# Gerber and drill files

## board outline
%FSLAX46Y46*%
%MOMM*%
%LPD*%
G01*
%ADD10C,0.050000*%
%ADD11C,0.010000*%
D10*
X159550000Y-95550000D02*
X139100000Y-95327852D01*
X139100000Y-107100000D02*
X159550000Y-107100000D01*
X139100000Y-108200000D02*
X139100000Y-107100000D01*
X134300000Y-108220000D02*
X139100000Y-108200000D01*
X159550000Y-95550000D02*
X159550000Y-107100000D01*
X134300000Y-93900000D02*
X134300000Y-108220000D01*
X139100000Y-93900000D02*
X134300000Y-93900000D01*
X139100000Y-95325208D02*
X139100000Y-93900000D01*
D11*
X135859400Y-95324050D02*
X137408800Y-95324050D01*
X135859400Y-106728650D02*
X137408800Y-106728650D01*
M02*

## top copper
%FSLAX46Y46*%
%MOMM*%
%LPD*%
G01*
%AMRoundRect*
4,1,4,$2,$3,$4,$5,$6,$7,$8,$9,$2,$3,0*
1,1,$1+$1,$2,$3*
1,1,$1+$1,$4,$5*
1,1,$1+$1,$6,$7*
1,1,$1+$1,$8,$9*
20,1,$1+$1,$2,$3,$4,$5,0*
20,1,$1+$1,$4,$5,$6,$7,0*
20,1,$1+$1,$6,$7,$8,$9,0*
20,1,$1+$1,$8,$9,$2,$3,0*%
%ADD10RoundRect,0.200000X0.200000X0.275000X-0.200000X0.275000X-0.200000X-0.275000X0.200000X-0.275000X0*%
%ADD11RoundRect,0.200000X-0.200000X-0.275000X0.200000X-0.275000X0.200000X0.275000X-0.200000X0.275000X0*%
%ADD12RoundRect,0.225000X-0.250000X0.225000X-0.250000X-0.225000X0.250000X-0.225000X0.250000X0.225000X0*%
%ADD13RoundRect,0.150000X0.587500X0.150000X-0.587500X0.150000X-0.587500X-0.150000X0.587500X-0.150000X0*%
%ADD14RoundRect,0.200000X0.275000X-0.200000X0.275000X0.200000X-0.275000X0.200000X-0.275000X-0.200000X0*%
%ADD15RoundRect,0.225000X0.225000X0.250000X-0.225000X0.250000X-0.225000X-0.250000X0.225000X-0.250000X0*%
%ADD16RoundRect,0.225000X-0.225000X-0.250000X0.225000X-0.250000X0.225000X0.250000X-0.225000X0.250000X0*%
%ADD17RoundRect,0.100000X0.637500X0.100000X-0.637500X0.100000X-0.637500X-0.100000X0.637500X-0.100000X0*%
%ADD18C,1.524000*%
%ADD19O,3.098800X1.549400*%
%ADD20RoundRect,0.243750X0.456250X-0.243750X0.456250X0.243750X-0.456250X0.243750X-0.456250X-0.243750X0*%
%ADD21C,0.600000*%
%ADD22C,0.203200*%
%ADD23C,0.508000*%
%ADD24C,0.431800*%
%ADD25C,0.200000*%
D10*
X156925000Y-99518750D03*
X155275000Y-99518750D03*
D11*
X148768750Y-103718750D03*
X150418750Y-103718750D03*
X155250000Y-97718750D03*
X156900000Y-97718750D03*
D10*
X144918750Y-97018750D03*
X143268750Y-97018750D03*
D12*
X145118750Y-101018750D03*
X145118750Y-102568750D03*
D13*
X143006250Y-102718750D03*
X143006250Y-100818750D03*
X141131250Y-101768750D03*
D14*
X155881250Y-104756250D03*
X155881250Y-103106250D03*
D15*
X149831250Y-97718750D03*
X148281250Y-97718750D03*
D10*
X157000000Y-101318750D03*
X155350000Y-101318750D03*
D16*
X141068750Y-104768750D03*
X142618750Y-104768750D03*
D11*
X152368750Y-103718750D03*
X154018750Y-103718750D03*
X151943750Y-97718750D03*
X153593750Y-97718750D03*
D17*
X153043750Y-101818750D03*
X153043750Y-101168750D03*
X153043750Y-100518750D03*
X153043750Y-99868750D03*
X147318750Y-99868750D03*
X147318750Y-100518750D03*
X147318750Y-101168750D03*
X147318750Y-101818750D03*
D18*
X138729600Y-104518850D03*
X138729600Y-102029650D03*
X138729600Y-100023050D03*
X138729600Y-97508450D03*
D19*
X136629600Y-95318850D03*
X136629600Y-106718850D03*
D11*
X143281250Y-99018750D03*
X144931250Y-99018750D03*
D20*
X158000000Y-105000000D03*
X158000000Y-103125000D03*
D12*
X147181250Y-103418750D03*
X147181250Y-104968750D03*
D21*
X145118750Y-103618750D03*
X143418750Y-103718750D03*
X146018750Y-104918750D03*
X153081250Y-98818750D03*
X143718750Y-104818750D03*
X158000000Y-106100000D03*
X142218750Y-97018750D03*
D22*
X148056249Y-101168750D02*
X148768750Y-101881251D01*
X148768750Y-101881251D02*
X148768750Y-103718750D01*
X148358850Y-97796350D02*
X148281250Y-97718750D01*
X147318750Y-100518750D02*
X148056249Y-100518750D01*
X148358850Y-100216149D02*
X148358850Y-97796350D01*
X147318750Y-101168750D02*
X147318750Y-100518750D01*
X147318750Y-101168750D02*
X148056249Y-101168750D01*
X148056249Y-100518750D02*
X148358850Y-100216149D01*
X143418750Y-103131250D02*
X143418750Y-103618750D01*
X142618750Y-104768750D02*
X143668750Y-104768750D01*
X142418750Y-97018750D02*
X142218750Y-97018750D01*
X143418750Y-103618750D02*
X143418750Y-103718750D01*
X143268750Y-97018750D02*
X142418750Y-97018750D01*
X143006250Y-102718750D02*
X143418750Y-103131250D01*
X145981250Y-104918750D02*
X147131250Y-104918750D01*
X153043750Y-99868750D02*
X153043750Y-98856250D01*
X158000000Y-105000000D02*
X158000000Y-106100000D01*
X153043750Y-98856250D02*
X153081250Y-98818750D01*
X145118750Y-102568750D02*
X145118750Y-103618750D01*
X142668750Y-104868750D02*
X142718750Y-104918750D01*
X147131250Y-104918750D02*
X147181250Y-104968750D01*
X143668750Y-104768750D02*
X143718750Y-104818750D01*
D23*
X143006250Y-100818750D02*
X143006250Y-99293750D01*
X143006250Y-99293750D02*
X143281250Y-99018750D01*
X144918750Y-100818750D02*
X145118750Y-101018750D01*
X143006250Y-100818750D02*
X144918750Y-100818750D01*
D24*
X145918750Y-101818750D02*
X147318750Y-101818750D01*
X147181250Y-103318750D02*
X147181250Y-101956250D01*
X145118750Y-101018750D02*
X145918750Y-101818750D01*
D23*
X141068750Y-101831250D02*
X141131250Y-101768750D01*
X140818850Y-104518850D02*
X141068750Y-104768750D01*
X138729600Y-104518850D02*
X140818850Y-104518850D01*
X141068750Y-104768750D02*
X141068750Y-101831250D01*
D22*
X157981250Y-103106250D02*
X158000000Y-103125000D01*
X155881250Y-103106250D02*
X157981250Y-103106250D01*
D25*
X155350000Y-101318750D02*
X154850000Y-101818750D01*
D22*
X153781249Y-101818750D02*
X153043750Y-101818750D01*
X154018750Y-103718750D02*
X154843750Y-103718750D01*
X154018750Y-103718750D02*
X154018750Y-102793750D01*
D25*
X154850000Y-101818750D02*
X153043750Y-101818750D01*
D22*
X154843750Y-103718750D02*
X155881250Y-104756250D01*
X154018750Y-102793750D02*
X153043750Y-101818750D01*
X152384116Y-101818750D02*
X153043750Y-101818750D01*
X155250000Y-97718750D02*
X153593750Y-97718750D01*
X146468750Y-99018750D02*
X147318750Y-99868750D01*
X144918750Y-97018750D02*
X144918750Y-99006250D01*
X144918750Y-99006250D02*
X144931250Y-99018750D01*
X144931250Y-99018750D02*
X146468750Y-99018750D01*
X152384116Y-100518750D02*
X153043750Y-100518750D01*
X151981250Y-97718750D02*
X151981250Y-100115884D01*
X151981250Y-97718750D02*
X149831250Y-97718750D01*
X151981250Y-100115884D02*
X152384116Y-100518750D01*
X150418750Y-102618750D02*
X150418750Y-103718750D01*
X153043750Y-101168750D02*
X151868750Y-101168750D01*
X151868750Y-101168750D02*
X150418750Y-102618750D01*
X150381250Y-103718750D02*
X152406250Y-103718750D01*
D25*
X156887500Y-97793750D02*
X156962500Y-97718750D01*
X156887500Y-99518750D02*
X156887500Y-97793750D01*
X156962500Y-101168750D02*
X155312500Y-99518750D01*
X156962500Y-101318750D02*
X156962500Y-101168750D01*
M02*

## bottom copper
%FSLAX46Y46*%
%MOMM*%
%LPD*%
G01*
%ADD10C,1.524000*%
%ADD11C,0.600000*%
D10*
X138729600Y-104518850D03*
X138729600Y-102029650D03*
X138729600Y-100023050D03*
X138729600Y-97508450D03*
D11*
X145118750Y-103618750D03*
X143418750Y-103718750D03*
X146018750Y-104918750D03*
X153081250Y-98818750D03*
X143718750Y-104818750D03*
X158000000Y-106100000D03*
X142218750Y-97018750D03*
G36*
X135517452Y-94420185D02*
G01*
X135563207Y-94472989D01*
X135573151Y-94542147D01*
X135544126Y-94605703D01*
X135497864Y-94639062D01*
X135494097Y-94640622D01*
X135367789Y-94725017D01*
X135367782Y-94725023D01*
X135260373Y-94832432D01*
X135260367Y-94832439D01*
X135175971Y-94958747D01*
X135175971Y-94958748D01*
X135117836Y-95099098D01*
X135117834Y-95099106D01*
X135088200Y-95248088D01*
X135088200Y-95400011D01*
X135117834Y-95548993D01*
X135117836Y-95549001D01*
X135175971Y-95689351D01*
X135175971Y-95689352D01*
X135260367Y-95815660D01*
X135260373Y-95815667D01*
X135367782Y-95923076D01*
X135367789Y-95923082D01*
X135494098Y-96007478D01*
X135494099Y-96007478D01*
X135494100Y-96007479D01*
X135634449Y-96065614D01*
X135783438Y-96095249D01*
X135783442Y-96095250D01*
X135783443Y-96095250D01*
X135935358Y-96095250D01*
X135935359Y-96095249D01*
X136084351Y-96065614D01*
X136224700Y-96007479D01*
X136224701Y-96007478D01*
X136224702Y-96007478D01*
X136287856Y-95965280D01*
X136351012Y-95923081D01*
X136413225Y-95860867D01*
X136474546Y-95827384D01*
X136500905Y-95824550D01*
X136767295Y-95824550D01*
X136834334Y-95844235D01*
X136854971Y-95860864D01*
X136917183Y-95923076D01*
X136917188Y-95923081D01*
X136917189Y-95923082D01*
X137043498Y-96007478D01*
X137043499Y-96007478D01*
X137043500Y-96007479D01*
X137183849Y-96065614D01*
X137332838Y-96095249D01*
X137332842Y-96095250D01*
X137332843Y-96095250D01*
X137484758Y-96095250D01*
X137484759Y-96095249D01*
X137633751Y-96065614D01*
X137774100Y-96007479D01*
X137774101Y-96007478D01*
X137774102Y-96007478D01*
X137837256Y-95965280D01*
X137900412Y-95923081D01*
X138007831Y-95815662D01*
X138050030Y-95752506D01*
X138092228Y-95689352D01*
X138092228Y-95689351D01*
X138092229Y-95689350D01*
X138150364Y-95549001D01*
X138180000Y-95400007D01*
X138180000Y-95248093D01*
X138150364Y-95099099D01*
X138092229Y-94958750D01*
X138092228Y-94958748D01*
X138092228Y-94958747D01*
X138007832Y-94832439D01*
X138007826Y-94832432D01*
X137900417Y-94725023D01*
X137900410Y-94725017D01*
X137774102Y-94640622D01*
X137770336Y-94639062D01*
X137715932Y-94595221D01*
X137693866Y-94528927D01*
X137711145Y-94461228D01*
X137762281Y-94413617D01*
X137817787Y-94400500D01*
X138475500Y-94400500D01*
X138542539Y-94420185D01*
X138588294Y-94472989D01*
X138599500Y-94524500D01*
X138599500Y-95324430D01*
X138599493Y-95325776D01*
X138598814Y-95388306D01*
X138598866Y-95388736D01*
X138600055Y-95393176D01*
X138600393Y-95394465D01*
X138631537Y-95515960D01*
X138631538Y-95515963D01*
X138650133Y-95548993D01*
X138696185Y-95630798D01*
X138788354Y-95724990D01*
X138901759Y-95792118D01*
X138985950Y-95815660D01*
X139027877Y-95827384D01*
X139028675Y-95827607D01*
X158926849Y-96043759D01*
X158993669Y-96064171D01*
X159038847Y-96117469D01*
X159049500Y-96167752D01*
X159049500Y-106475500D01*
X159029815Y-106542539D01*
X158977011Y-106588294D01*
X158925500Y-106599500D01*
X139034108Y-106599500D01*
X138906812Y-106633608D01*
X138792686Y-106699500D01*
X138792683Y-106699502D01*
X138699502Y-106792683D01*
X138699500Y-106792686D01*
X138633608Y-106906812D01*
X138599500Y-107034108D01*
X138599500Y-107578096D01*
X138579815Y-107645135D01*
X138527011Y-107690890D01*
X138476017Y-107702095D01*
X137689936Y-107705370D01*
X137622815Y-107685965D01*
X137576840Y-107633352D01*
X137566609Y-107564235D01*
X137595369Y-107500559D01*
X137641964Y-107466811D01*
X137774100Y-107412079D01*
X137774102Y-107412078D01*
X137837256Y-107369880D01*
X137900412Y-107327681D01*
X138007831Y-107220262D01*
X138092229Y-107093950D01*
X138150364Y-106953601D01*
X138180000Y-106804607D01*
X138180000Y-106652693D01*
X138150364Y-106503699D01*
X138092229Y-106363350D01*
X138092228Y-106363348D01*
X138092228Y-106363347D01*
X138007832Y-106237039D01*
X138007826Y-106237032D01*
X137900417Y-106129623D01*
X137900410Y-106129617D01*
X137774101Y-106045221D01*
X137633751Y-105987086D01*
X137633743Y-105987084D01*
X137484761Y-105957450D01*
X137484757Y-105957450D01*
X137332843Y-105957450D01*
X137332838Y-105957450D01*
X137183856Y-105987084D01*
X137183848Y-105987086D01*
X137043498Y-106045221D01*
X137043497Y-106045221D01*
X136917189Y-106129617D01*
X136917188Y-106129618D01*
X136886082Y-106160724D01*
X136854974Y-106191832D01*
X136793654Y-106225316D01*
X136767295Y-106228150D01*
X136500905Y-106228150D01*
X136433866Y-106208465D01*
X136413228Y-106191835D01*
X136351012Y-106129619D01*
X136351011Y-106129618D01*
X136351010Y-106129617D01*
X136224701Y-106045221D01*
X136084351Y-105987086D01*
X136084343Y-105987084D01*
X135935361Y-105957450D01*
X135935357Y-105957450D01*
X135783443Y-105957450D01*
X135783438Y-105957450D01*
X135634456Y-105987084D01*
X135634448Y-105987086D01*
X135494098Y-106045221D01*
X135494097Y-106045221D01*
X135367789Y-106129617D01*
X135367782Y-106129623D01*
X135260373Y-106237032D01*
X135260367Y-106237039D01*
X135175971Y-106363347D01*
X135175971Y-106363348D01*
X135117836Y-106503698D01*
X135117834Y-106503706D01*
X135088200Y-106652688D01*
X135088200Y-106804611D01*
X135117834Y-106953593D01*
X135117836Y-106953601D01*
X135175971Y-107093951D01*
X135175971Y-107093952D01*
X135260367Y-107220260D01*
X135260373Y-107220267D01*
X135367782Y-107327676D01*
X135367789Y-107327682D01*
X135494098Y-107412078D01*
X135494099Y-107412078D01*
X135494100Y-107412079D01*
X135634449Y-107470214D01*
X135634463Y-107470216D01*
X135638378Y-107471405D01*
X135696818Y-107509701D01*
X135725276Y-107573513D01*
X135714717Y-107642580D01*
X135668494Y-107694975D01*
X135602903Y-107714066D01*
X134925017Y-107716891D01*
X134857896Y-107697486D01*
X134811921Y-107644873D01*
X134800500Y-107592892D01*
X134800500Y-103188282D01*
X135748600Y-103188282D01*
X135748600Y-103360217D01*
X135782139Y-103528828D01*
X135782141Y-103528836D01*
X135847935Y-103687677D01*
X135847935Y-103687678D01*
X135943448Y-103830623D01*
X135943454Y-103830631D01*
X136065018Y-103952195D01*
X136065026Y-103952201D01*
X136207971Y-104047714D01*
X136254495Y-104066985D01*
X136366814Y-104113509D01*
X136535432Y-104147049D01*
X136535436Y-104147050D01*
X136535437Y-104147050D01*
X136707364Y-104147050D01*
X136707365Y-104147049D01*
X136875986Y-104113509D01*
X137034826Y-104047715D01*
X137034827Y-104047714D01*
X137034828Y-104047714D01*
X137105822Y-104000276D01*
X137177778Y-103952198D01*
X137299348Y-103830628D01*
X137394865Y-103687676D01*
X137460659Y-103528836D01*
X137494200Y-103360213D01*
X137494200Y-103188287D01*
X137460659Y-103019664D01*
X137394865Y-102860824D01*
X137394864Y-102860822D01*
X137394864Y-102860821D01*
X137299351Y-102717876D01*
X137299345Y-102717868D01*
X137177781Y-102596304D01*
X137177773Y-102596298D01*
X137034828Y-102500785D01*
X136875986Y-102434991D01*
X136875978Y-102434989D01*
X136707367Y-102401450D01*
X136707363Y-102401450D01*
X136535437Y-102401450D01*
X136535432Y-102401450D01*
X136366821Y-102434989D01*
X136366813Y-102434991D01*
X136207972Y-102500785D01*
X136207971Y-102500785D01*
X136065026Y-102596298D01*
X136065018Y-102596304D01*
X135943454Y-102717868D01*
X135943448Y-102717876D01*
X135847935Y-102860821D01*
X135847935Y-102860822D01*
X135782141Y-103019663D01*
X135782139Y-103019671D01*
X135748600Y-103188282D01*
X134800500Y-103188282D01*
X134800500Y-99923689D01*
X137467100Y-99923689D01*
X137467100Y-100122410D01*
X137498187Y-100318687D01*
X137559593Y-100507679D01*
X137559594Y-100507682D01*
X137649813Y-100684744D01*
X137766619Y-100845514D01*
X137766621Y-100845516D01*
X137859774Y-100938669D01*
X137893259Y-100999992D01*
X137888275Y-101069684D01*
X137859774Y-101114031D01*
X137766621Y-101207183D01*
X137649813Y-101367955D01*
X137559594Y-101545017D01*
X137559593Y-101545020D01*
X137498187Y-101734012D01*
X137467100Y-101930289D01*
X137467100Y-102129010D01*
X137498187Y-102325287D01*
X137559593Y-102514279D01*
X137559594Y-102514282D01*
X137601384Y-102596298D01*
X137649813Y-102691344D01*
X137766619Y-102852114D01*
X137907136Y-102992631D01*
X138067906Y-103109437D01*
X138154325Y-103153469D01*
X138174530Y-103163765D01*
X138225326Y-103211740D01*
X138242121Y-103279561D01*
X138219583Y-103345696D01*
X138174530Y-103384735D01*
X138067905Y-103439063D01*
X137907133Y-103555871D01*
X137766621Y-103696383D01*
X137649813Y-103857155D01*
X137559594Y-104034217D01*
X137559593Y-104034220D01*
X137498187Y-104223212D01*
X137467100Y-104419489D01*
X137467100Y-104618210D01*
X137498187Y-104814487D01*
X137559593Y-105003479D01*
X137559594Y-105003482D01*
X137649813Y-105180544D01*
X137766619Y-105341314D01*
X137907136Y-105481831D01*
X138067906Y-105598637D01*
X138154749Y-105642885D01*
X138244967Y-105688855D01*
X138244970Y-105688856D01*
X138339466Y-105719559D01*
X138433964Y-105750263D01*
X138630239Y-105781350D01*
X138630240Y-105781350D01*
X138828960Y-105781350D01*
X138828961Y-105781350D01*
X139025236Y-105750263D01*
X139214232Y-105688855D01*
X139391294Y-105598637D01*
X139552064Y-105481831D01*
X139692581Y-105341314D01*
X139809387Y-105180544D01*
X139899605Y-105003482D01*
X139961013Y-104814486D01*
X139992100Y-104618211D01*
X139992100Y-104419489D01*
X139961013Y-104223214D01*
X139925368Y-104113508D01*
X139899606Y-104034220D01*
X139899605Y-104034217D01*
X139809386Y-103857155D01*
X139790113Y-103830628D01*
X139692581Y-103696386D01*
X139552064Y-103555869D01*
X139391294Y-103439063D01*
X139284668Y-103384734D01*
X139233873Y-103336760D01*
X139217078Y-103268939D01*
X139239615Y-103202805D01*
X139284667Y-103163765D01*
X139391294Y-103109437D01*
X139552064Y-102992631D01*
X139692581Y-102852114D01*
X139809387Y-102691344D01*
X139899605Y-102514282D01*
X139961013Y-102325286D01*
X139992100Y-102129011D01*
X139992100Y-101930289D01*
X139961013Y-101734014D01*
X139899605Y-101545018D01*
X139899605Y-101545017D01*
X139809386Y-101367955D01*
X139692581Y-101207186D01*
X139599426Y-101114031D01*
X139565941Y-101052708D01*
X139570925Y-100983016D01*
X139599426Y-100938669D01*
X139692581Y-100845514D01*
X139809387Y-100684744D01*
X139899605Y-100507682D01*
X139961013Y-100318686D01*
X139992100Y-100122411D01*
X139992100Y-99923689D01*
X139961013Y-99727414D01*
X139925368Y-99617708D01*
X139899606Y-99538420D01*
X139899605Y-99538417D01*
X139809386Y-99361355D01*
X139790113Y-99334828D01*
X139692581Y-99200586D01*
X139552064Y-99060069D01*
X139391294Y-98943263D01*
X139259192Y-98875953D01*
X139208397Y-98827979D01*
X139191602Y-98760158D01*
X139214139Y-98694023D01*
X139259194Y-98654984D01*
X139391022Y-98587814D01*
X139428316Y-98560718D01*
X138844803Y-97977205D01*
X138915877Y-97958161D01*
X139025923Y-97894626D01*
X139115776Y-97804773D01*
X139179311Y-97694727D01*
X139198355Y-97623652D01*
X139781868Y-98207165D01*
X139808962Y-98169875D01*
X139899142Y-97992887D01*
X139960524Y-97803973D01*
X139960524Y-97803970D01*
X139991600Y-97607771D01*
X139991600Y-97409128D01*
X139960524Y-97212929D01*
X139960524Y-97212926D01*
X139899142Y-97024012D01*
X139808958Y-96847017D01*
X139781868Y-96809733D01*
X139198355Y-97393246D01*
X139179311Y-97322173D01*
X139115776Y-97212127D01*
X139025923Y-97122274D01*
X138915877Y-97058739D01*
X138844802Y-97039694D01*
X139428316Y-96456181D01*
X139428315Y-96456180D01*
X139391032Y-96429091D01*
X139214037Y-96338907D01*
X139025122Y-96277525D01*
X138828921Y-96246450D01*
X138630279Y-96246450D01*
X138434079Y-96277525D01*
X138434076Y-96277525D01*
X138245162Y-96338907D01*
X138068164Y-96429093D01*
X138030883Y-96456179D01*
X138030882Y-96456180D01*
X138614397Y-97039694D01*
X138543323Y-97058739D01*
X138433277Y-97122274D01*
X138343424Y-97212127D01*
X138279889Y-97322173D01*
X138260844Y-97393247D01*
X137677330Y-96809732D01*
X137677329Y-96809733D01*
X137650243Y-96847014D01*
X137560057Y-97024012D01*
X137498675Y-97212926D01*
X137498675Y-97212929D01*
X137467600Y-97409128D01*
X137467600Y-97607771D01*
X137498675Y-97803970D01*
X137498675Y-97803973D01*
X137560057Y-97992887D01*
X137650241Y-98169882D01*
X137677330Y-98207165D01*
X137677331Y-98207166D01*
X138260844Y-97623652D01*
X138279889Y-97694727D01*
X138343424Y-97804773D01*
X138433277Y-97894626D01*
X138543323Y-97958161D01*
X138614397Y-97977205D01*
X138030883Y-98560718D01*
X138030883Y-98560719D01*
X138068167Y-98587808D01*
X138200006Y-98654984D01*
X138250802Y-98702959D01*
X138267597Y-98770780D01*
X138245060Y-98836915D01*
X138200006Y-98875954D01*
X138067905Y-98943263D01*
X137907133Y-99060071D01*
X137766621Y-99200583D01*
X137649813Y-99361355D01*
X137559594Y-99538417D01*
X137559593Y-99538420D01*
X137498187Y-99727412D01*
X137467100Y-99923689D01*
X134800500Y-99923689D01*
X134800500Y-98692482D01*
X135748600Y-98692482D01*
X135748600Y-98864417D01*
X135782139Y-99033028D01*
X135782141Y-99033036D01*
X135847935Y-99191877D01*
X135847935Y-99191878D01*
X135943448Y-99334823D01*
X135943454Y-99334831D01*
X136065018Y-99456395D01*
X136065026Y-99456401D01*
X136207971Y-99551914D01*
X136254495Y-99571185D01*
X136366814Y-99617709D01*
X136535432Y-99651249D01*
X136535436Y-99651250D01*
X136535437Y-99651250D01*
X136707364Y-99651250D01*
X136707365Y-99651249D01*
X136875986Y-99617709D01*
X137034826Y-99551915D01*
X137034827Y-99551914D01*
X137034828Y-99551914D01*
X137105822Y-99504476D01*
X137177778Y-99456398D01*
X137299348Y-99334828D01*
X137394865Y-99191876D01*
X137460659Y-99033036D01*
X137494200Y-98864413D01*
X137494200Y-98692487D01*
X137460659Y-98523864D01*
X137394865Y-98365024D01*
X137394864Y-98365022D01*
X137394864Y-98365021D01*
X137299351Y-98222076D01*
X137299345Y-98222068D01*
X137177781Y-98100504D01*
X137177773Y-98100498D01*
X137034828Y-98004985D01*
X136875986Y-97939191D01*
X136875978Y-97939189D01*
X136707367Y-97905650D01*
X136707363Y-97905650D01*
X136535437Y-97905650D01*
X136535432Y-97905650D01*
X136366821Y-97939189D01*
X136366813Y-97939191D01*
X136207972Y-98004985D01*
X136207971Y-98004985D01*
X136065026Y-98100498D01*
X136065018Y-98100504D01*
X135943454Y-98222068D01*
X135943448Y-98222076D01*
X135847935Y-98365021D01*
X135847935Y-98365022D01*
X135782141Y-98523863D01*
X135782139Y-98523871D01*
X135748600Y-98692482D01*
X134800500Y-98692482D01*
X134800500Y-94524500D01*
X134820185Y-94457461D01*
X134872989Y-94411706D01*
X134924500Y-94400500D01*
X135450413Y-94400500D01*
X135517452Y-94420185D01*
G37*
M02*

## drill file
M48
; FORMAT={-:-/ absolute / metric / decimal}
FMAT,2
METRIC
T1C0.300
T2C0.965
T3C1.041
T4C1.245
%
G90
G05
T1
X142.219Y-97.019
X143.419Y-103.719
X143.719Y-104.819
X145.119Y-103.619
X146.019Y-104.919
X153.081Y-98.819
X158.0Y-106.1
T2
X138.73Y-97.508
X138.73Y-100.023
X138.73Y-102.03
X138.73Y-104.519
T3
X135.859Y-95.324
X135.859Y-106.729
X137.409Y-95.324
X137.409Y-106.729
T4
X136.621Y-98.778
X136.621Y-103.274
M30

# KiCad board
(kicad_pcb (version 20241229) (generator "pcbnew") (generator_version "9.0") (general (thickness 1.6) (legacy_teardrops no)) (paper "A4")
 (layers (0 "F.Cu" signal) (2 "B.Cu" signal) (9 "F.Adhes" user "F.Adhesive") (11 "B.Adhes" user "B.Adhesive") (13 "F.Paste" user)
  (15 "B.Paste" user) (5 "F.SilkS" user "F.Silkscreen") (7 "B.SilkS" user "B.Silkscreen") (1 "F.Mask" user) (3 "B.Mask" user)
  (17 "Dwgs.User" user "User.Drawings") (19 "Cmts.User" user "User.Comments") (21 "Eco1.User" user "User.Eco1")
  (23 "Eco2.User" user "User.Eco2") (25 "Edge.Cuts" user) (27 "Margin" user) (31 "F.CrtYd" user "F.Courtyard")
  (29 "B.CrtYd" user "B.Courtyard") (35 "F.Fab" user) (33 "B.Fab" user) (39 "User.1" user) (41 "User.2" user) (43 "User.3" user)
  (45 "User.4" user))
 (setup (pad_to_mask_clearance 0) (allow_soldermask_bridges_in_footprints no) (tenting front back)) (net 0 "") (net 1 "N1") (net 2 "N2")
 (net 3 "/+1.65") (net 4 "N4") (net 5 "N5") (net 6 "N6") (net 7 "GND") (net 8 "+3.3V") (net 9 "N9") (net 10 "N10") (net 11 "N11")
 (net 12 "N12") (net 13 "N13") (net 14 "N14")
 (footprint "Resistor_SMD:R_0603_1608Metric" (layer "F.Cu") (at 156.1 99.51875 180)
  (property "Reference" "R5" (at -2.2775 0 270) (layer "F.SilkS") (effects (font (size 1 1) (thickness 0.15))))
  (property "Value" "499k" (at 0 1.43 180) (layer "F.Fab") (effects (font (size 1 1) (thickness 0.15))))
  (pad "1" smd roundrect (at -0.825 0 180) (size 0.8 0.95) (layers "F.Cu" "F.Mask" "F.Paste") (roundrect_rratio 0.25) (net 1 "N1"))
  (pad "2" smd roundrect (at 0.825 0 180) (size 0.8 0.95) (layers "F.Cu" "F.Mask" "F.Paste") (roundrect_rratio 0.25) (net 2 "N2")))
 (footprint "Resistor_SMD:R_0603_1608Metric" (layer "F.Cu") (at 149.59375 103.71875)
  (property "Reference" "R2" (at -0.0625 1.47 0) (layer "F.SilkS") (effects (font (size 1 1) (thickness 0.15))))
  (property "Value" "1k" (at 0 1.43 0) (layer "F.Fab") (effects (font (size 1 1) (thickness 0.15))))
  (pad "1" smd roundrect (at -0.825 0) (size 0.8 0.95) (layers "F.Cu" "F.Mask" "F.Paste") (roundrect_rratio 0.25) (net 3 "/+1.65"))
  (pad "2" smd roundrect (at 0.825 0) (size 0.8 0.95) (layers "F.Cu" "F.Mask" "F.Paste") (roundrect_rratio 0.25) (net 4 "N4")))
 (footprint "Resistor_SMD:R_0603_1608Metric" (layer "F.Cu") (at 156.075 97.71875)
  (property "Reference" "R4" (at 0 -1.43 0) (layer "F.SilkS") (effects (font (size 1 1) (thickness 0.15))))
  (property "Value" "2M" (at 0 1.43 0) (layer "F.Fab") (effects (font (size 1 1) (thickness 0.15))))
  (pad "1" smd roundrect (at -0.825 0) (size 0.8 0.95) (layers "F.Cu" "F.Mask" "F.Paste") (roundrect_rratio 0.25) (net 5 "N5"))
  (pad "2" smd roundrect (at 0.825 0) (size 0.8 0.95) (layers "F.Cu" "F.Mask" "F.Paste") (roundrect_rratio 0.25) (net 1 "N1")))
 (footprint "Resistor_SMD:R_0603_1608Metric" (layer "F.Cu") (at 144.09375 97.01875 180)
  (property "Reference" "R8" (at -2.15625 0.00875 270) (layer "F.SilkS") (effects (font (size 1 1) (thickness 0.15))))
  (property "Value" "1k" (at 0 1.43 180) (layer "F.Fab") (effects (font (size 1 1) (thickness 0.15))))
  (pad "1" smd roundrect (at -0.825 0 180) (size 0.8 0.95) (layers "F.Cu" "F.Mask" "F.Paste") (roundrect_rratio 0.25) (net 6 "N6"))
  (pad "2" smd roundrect (at 0.825 0 180) (size 0.8 0.95) (layers "F.Cu" "F.Mask" "F.Paste") (roundrect_rratio 0.25) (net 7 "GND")))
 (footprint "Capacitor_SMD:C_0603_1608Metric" (layer "F.Cu") (at 145.11875 101.79375 -90)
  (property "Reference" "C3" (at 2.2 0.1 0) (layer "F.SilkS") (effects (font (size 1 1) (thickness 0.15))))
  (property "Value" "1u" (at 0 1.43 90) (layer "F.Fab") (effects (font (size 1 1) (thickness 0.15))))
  (pad "1" smd roundrect (at -0.775 0 270) (size 0.9 0.95) (layers "F.Cu" "F.Mask" "F.Paste") (roundrect_rratio 0.25) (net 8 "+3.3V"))
  (pad "2" smd roundrect (at 0.775 0 270) (size 0.9 0.95) (layers "F.Cu" "F.Mask" "F.Paste") (roundrect_rratio 0.25) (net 7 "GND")))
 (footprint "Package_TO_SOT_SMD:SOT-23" (layer "F.Cu") (at 142.06875 101.76875 180)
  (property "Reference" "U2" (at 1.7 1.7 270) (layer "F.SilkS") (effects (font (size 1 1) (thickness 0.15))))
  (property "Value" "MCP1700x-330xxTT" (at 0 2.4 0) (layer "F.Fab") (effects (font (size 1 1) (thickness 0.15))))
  (pad "1" smd roundrect (at -0.9375 -0.95 180) (size 1.475 0.6) (layers "F.Cu" "F.Mask" "F.Paste") (roundrect_rratio 0.25) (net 7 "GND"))
  (pad "2" smd roundrect (at -0.9375 0.95 180) (size 1.475 0.6) (layers "F.Cu" "F.Mask" "F.Paste") (roundrect_rratio 0.25) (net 8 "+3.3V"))
  (pad "3" smd roundrect (at 0.9375 0 180) (size 1.475 0.6) (layers "F.Cu" "F.Mask" "F.Paste") (roundrect_rratio 0.25) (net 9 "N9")))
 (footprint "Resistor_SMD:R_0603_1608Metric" (layer "F.Cu") (at 155.88125 103.93125 90)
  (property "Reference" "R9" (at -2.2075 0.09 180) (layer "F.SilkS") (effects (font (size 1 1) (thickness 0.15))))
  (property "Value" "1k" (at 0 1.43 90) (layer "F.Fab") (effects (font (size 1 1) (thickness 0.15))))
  (pad "1" smd roundrect (at -0.825 0 90) (size 0.8 0.95) (layers "F.Cu" "F.Mask" "F.Paste") (roundrect_rratio 0.25) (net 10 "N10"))
  (pad "2" smd roundrect (at 0.825 0 90) (size 0.8 0.95) (layers "F.Cu" "F.Mask" "F.Paste") (roundrect_rratio 0.25) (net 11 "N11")))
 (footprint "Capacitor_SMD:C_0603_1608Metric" (layer "F.Cu") (at 149.05625 97.71875 180)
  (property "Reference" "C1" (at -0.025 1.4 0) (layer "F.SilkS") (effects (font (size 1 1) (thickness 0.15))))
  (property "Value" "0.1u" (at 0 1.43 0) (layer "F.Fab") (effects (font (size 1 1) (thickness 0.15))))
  (pad "1" smd roundrect (at -0.775 0 180) (size 0.9 0.95) (layers "F.Cu" "F.Mask" "F.Paste") (roundrect_rratio 0.25) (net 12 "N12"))
  (pad "2" smd roundrect (at 0.775 0 180) (size 0.9 0.95) (layers "F.Cu" "F.Mask" "F.Paste") (roundrect_rratio 0.25) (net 3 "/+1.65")))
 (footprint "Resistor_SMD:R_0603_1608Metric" (layer "F.Cu") (at 156.175 101.31875 180)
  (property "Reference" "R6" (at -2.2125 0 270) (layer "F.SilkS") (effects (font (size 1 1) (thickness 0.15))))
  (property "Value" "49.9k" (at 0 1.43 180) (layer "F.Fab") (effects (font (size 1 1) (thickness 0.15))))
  (pad "1" smd roundrect (at -0.825 0 180) (size 0.8 0.95) (layers "F.Cu" "F.Mask" "F.Paste") (roundrect_rratio 0.25) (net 2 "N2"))
  (pad "2" smd roundrect (at 0.825 0 180) (size 0.8 0.95) (layers "F.Cu" "F.Mask" "F.Paste") (roundrect_rratio 0.25) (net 10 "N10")))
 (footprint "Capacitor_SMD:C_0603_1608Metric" (layer "F.Cu") (at 141.84375 104.76875)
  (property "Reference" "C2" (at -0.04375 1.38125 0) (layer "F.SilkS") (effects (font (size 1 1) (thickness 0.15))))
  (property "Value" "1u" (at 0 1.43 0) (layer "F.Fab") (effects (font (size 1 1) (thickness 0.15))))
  (pad "1" smd roundrect (at -0.775 0) (size 0.9 0.95) (layers "F.Cu" "F.Mask" "F.Paste") (roundrect_rratio 0.25) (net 9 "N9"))
  (pad "2" smd roundrect (at 0.775 0) (size 0.9 0.95) (layers "F.Cu" "F.Mask" "F.Paste") (roundrect_rratio 0.25) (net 7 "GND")))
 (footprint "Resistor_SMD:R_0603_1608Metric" (layer "F.Cu") (at 153.19375 103.71875)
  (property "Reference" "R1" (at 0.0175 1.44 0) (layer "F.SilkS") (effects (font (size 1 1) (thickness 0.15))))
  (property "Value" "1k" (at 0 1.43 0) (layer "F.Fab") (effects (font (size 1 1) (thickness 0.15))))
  (pad "1" smd roundrect (at -0.825 0) (size 0.8 0.95) (layers "F.Cu" "F.Mask" "F.Paste") (roundrect_rratio 0.25) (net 4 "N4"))
  (pad "2" smd roundrect (at 0.825 0) (size 0.8 0.95) (layers "F.Cu" "F.Mask" "F.Paste") (roundrect_rratio 0.25) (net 10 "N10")))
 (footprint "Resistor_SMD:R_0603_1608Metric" (layer "F.Cu") (at 152.76875 97.71875)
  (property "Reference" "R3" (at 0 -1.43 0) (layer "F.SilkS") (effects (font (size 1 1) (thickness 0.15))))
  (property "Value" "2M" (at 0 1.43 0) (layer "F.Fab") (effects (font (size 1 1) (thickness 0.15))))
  (pad "1" smd roundrect (at -0.825 0) (size 0.8 0.95) (layers "F.Cu" "F.Mask" "F.Paste") (roundrect_rratio 0.25) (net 12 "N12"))
  (pad "2" smd roundrect (at 0.825 0) (size 0.8 0.95) (layers "F.Cu" "F.Mask" "F.Paste") (roundrect_rratio 0.25) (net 5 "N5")))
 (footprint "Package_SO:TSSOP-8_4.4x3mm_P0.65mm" (layer "F.Cu") (at 150.18125 100.84375 180)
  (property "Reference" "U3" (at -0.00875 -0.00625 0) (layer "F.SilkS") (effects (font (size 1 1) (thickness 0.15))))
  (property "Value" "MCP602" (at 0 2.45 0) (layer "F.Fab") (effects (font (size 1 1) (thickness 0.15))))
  (pad "1" smd roundrect (at -2.8625 -0.975 180) (size 1.475 0.4) (layers "F.Cu" "F.Mask" "F.Paste") (roundrect_rratio 0.25) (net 10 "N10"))
  (pad "2" smd roundrect (at -2.8625 -0.325 180) (size 1.475 0.4) (layers "F.Cu" "F.Mask" "F.Paste") (roundrect_rratio 0.25) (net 4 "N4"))
  (pad "3" smd roundrect (at -2.8625 0.325 180) (size 1.475 0.4) (layers "F.Cu" "F.Mask" "F.Paste") (roundrect_rratio 0.25) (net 12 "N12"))
  (pad "4" smd roundrect (at -2.8625 0.975 180) (size 1.475 0.4) (layers "F.Cu" "F.Mask" "F.Paste") (roundrect_rratio 0.25) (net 7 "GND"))
  (pad "5" smd roundrect (at 2.8625 0.975 180) (size 1.475 0.4) (layers "F.Cu" "F.Mask" "F.Paste") (roundrect_rratio 0.25) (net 6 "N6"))
  (pad "6" smd roundrect (at 2.8625 0.325 180) (size 1.475 0.4) (layers "F.Cu" "F.Mask" "F.Paste") (roundrect_rratio 0.25) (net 3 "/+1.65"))
  (pad "7" smd roundrect (at 2.8625 -0.325 180) (size 1.475 0.4) (layers "F.Cu" "F.Mask" "F.Paste") (roundrect_rratio 0.25) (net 3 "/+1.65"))
  (pad "8" smd roundrect (at 2.8625 -0.975 180) (size 1.475 0.4) (layers "F.Cu" "F.Mask" "F.Paste") (roundrect_rratio 0.25) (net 8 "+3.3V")))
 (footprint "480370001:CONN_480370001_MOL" (layer "F.Cu") (at 138.7296 104.51885 -90)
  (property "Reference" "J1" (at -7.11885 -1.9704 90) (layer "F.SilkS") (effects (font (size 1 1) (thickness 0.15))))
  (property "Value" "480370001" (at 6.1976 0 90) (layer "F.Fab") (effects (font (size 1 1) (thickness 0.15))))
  (fp_line (start -9.1948 2.8702) (end -9.1948 1.3208) (stroke (width 0.01) (type solid)) (layer "Edge.Cuts"))
  (fp_line (start 2.2098 2.8702) (end 2.2098 1.3208) (stroke (width 0.01) (type solid)) (layer "Edge.Cuts"))
  (pad "" np_thru_hole circle (at -9.1948 1.3208 270) (size 1.0414 1.0414) (drill 1.0414) (layers "*.Cu" "*.Mask"))
  (pad "" np_thru_hole circle (at -9.1948 2.8702 270) (size 1.0414 1.0414) (drill 1.0414) (layers "*.Cu" "*.Mask"))
  (pad "" np_thru_hole circle (at -5.7404 2.1082 270) (size 1.2446 1.2446) (drill 1.2446) (layers "*.Cu" "*.Mask"))
  (pad "" np_thru_hole circle (at -1.2446 2.1082 270) (size 1.2446 1.2446) (drill 1.2446) (layers "*.Cu" "*.Mask"))
  (pad "" np_thru_hole circle (at 2.2098 1.3208 270) (size 1.0414 1.0414) (drill 1.0414) (layers "*.Cu" "*.Mask"))
  (pad "" np_thru_hole circle (at 2.2098 2.8702 270) (size 1.0414 1.0414) (drill 1.0414) (layers "*.Cu" "*.Mask"))
  (pad "1" thru_hole circle (at 0 0 270) (size 1.524 1.524) (drill 0.9652) (layers "*.Cu" "*.Mask") (remove_unused_layers no) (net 9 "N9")
   (solder_mask_margin 0.102))
  (pad "2" thru_hole circle (at -2.4892 0 270) (size 1.524 1.524) (drill 0.9652) (layers "*.Cu" "*.Mask") (remove_unused_layers no)
   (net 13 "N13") (solder_mask_margin 0.102))
  (pad "3" thru_hole circle (at -4.4958 0 270) (size 1.524 1.524) (drill 0.9652) (layers "*.Cu" "*.Mask") (remove_unused_layers no)
   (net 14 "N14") (solder_mask_margin 0.102))
  (pad "4" thru_hole circle (at -7.0104 0 270) (size 1.524 1.524) (drill 0.9652) (layers "*.Cu" "*.Mask") (remove_unused_layers no)
   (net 7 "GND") (solder_mask_margin 0.102))
  (pad "7" smd oval (at -9.2 2.1 270) (size 1.5494 3.0988) (layers "F.Cu" "F.Mask" "F.Paste") (solder_mask_margin 0.102))
  (pad "8" smd oval (at 2.2 2.1 270) (size 1.5494 3.0988) (layers "F.Cu" "F.Mask" "F.Paste") (solder_mask_margin 0.102)))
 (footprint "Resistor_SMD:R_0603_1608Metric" (layer "F.Cu") (at 144.10625 99.01875)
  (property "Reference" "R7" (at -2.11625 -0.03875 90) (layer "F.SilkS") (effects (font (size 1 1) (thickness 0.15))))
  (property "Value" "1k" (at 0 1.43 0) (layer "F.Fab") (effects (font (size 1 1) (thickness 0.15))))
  (pad "1" smd roundrect (at -0.825 0) (size 0.8 0.95) (layers "F.Cu" "F.Mask" "F.Paste") (roundrect_rratio 0.25) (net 8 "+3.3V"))
  (pad "2" smd roundrect (at 0.825 0) (size 0.8 0.95) (layers "F.Cu" "F.Mask" "F.Paste") (roundrect_rratio 0.25) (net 6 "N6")))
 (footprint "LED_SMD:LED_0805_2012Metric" (layer "F.Cu") (at 158 104.0625 90)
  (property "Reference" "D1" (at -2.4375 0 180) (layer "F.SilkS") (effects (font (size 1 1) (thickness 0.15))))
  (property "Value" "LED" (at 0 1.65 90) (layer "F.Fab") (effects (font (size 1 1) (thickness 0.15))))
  (pad "1" smd roundrect (at -0.9375 0 90) (size 0.975 1.4) (layers "F.Cu" "F.Mask" "F.Paste") (roundrect_rratio 0.25) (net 7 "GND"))
  (pad "2" smd roundrect (at 0.9375 0 90) (size 0.975 1.4) (layers "F.Cu" "F.Mask" "F.Paste") (roundrect_rratio 0.25) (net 11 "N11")))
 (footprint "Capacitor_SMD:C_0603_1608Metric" (layer "F.Cu") (at 147.18125 104.19375 -90)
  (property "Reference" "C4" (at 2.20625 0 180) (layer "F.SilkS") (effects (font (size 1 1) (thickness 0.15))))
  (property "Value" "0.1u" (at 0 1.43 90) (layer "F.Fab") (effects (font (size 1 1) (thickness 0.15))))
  (pad "1" smd roundrect (at -0.775 0 270) (size 0.9 0.95) (layers "F.Cu" "F.Mask" "F.Paste") (roundrect_rratio 0.25) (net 8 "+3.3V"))
  (pad "2" smd roundrect (at 0.775 0 270) (size 0.9 0.95) (layers "F.Cu" "F.Mask" "F.Paste") (roundrect_rratio 0.25) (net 7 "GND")))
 (gr_line (start 159.55 95.55) (end 139.1 95.327852) (stroke (width 0.05) (type default)) (layer "Edge.Cuts"))
 (gr_line (start 139.1 107.1) (end 159.55 107.1) (stroke (width 0.05) (type default)) (layer "Edge.Cuts"))
 (gr_line (start 139.1 108.2) (end 139.1 107.1) (stroke (width 0.05) (type default)) (layer "Edge.Cuts"))
 (gr_line (start 134.3 108.22) (end 139.1 108.2) (stroke (width 0.05) (type default)) (layer "Edge.Cuts"))
 (gr_line (start 159.55 95.55) (end 159.55 107.1) (stroke (width 0.05) (type default)) (layer "Edge.Cuts"))
 (gr_line (start 134.3 93.9) (end 134.3 108.22) (stroke (width 0.05) (type default)) (layer "Edge.Cuts"))
 (gr_line (start 139.1 93.9) (end 134.3 93.9) (stroke (width 0.05) (type default)) (layer "Edge.Cuts"))
 (gr_line (start 139.1 95.325208) (end 139.1 93.9) (stroke (width 0.05) (type default)) (layer "Edge.Cuts"))
 (segment (start 148.056249 101.16875) (end 148.76875 101.881251) (width 0.2032) (layer "F.Cu") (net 3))
 (segment (start 148.76875 101.881251) (end 148.76875 103.71875) (width 0.2032) (layer "F.Cu") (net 3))
 (segment (start 148.35885 97.79635) (end 148.28125 97.71875) (width 0.2032) (layer "F.Cu") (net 3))
 (segment (start 147.31875 100.51875) (end 148.056249 100.51875) (width 0.2032) (layer "F.Cu") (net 3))
 (segment (start 148.35885 100.216149) (end 148.35885 97.79635) (width 0.2032) (layer "F.Cu") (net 3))
 (segment (start 147.31875 101.16875) (end 147.31875 100.51875) (width 0.2032) (layer "F.Cu") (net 3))
 (segment (start 147.31875 101.16875) (end 148.056249 101.16875) (width 0.2032) (layer "F.Cu") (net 3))
 (segment (start 148.056249 100.51875) (end 148.35885 100.216149) (width 0.2032) (layer "F.Cu") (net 3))
 (segment (start 143.41875 103.13125) (end 143.41875 103.61875) (width 0.2032) (layer "F.Cu") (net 7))
 (segment (start 142.61875 104.76875) (end 143.66875 104.76875) (width 0.2032) (layer "F.Cu") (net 7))
 (segment (start 142.41875 97.01875) (end 142.21875 97.01875) (width 0.2032) (layer "F.Cu") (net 7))
 (segment (start 143.41875 103.61875) (end 143.41875 103.71875) (width 0.2032) (layer "F.Cu") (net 7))
 (segment (start 143.26875 97.01875) (end 142.41875 97.01875) (width 0.2032) (layer "F.Cu") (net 7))
 (segment (start 143.00625 102.71875) (end 143.41875 103.13125) (width 0.2032) (layer "F.Cu") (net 7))
 (segment (start 145.98125 104.91875) (end 147.13125 104.91875) (width 0.2032) (layer "F.Cu") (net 7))
 (segment (start 153.04375 99.86875) (end 153.04375 98.85625) (width 0.2032) (layer "F.Cu") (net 7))
 (segment (start 158 105) (end 158 106.1) (width 0.2032) (layer "F.Cu") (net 7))
 (segment (start 153.04375 98.85625) (end 153.08125 98.81875) (width 0.2032) (layer "F.Cu") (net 7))
 (segment (start 145.11875 102.56875) (end 145.11875 103.61875) (width 0.2032) (layer "F.Cu") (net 7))
 (segment (start 142.66875 104.86875) (end 142.71875 104.91875) (width 0.2032) (layer "F.Cu") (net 7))
 (segment (start 147.13125 104.91875) (end 147.18125 104.96875) (width 0.2032) (layer "F.Cu") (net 7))
 (segment (start 143.66875 104.76875) (end 143.71875 104.81875) (width 0.2032) (layer "F.Cu") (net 7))
 (via (at 145.11875 103.61875) (size 0.6) (drill 0.3) (layers "F.Cu" "B.Cu") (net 7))
 (via (at 143.41875 103.71875) (size 0.6) (drill 0.3) (layers "F.Cu" "B.Cu") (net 7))
 (via (at 146.01875 104.91875) (size 0.6) (drill 0.3) (layers "F.Cu" "B.Cu") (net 7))
 (via (at 153.08125 98.81875) (size 0.6) (drill 0.3) (layers "F.Cu" "B.Cu") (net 7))
 (via (at 143.71875 104.81875) (size 0.6) (drill 0.3) (layers "F.Cu" "B.Cu") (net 7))
 (via (at 158 106.1) (size 0.6) (drill 0.3) (layers "F.Cu" "B.Cu") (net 7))
 (via (at 142.21875 97.01875) (size 0.6) (drill 0.3) (layers "F.Cu" "B.Cu") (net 7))
 (segment (start 143.00625 100.81875) (end 143.00625 99.29375) (width 0.508) (layer "F.Cu") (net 8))
 (segment (start 143.00625 99.29375) (end 143.28125 99.01875) (width 0.508) (layer "F.Cu") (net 8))
 (segment (start 144.91875 100.81875) (end 145.11875 101.01875) (width 0.508) (layer "F.Cu") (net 8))
 (segment (start 143.00625 100.81875) (end 144.91875 100.81875) (width 0.508) (layer "F.Cu") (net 8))
 (segment (start 145.91875 101.81875) (end 147.31875 101.81875) (width 0.4318) (layer "F.Cu") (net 8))
 (segment (start 147.18125 103.31875) (end 147.18125 101.95625) (width 0.4318) (layer "F.Cu") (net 8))
 (segment (start 145.11875 101.01875) (end 145.91875 101.81875) (width 0.4318) (layer "F.Cu") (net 8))
 (segment (start 141.06875 101.83125) (end 141.13125 101.76875) (width 0.508) (layer "F.Cu") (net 9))
 (segment (start 140.81885 104.51885) (end 141.06875 104.76875) (width 0.508) (layer "F.Cu") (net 9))
 (segment (start 138.7296 104.51885) (end 140.81885 104.51885) (width 0.508) (layer "F.Cu") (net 9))
 (segment (start 141.06875 104.76875) (end 141.06875 101.83125) (width 0.508) (layer "F.Cu") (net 9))
 (segment (start 157.98125 103.10625) (end 158 103.125) (width 0.2032) (layer "F.Cu") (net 11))
 (segment (start 155.88125 103.10625) (end 157.98125 103.10625) (width 0.2032) (layer "F.Cu") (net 11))
 (segment (start 155.35 101.31875) (end 154.85 101.81875) (width 0.2) (layer "F.Cu") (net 10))
 (segment (start 153.781249 101.81875) (end 153.04375 101.81875) (width 0.2032) (layer "F.Cu") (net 10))
 (segment (start 154.01875 103.71875) (end 154.84375 103.71875) (width 0.2032) (layer "F.Cu") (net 10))
 (segment (start 154.01875 103.71875) (end 154.01875 102.79375) (width 0.2032) (layer "F.Cu") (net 10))
 (segment (start 154.85 101.81875) (end 153.04375 101.81875) (width 0.2) (layer "F.Cu") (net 10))
 (segment (start 154.84375 103.71875) (end 155.88125 104.75625) (width 0.2032) (layer "F.Cu") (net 10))
 (segment (start 154.01875 102.79375) (end 153.04375 101.81875) (width 0.2032) (layer "F.Cu") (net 10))
 (segment (start 152.384116 101.81875) (end 153.04375 101.81875) (width 0.2032) (layer "F.Cu") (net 10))
 (segment (start 155.25 97.71875) (end 153.59375 97.71875) (width 0.2032) (layer "F.Cu") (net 5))
 (segment (start 146.46875 99.01875) (end 147.31875 99.86875) (width 0.2032) (layer "F.Cu") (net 6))
 (segment (start 144.91875 97.01875) (end 144.91875 99.00625) (width 0.2032) (layer "F.Cu") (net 6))
 (segment (start 144.91875 99.00625) (end 144.93125 99.01875) (width 0.2032) (layer "F.Cu") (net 6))
 (segment (start 144.93125 99.01875) (end 146.46875 99.01875) (width 0.2032) (layer "F.Cu") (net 6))
 (segment (start 152.384116 100.51875) (end 153.04375 100.51875) (width 0.2032) (layer "F.Cu") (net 12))
 (segment (start 151.98125 97.71875) (end 151.98125 100.115884) (width 0.2032) (layer "F.Cu") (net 12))
 (segment (start 151.98125 97.71875) (end 149.83125 97.71875) (width 0.2032) (layer "F.Cu") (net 12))
 (segment (start 151.98125 100.115884) (end 152.384116 100.51875) (width 0.2032) (layer "F.Cu") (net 12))
 (segment (start 150.41875 102.61875) (end 150.41875 103.71875) (width 0.2032) (layer "F.Cu") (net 4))
 (segment (start 153.04375 101.16875) (end 151.86875 101.16875) (width 0.2032) (layer "F.Cu") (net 4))
 (segment (start 151.86875 101.16875) (end 150.41875 102.61875) (width 0.2032) (layer "F.Cu") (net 4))
 (segment (start 150.38125 103.71875) (end 152.40625 103.71875) (width 0.2032) (layer "F.Cu") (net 4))
 (segment (start 156.8875 97.79375) (end 156.9625 97.71875) (width 0.2) (layer "F.Cu") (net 1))
 (segment (start 156.8875 99.51875) (end 156.8875 97.79375) (width 0.2) (layer "F.Cu") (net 1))
 (segment (start 156.9625 101.16875) (end 155.3125 99.51875) (width 0.2) (layer "F.Cu") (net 2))
 (segment (start 156.9625 101.31875) (end 156.9625 101.16875) (width 0.2) (layer "F.Cu") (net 2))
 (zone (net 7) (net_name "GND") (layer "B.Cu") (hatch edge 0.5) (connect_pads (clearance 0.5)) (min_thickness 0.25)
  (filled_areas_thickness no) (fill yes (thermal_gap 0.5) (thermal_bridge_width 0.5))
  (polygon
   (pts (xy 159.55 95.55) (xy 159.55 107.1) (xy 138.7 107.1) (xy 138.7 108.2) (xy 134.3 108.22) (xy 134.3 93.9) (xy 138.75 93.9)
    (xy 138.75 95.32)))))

